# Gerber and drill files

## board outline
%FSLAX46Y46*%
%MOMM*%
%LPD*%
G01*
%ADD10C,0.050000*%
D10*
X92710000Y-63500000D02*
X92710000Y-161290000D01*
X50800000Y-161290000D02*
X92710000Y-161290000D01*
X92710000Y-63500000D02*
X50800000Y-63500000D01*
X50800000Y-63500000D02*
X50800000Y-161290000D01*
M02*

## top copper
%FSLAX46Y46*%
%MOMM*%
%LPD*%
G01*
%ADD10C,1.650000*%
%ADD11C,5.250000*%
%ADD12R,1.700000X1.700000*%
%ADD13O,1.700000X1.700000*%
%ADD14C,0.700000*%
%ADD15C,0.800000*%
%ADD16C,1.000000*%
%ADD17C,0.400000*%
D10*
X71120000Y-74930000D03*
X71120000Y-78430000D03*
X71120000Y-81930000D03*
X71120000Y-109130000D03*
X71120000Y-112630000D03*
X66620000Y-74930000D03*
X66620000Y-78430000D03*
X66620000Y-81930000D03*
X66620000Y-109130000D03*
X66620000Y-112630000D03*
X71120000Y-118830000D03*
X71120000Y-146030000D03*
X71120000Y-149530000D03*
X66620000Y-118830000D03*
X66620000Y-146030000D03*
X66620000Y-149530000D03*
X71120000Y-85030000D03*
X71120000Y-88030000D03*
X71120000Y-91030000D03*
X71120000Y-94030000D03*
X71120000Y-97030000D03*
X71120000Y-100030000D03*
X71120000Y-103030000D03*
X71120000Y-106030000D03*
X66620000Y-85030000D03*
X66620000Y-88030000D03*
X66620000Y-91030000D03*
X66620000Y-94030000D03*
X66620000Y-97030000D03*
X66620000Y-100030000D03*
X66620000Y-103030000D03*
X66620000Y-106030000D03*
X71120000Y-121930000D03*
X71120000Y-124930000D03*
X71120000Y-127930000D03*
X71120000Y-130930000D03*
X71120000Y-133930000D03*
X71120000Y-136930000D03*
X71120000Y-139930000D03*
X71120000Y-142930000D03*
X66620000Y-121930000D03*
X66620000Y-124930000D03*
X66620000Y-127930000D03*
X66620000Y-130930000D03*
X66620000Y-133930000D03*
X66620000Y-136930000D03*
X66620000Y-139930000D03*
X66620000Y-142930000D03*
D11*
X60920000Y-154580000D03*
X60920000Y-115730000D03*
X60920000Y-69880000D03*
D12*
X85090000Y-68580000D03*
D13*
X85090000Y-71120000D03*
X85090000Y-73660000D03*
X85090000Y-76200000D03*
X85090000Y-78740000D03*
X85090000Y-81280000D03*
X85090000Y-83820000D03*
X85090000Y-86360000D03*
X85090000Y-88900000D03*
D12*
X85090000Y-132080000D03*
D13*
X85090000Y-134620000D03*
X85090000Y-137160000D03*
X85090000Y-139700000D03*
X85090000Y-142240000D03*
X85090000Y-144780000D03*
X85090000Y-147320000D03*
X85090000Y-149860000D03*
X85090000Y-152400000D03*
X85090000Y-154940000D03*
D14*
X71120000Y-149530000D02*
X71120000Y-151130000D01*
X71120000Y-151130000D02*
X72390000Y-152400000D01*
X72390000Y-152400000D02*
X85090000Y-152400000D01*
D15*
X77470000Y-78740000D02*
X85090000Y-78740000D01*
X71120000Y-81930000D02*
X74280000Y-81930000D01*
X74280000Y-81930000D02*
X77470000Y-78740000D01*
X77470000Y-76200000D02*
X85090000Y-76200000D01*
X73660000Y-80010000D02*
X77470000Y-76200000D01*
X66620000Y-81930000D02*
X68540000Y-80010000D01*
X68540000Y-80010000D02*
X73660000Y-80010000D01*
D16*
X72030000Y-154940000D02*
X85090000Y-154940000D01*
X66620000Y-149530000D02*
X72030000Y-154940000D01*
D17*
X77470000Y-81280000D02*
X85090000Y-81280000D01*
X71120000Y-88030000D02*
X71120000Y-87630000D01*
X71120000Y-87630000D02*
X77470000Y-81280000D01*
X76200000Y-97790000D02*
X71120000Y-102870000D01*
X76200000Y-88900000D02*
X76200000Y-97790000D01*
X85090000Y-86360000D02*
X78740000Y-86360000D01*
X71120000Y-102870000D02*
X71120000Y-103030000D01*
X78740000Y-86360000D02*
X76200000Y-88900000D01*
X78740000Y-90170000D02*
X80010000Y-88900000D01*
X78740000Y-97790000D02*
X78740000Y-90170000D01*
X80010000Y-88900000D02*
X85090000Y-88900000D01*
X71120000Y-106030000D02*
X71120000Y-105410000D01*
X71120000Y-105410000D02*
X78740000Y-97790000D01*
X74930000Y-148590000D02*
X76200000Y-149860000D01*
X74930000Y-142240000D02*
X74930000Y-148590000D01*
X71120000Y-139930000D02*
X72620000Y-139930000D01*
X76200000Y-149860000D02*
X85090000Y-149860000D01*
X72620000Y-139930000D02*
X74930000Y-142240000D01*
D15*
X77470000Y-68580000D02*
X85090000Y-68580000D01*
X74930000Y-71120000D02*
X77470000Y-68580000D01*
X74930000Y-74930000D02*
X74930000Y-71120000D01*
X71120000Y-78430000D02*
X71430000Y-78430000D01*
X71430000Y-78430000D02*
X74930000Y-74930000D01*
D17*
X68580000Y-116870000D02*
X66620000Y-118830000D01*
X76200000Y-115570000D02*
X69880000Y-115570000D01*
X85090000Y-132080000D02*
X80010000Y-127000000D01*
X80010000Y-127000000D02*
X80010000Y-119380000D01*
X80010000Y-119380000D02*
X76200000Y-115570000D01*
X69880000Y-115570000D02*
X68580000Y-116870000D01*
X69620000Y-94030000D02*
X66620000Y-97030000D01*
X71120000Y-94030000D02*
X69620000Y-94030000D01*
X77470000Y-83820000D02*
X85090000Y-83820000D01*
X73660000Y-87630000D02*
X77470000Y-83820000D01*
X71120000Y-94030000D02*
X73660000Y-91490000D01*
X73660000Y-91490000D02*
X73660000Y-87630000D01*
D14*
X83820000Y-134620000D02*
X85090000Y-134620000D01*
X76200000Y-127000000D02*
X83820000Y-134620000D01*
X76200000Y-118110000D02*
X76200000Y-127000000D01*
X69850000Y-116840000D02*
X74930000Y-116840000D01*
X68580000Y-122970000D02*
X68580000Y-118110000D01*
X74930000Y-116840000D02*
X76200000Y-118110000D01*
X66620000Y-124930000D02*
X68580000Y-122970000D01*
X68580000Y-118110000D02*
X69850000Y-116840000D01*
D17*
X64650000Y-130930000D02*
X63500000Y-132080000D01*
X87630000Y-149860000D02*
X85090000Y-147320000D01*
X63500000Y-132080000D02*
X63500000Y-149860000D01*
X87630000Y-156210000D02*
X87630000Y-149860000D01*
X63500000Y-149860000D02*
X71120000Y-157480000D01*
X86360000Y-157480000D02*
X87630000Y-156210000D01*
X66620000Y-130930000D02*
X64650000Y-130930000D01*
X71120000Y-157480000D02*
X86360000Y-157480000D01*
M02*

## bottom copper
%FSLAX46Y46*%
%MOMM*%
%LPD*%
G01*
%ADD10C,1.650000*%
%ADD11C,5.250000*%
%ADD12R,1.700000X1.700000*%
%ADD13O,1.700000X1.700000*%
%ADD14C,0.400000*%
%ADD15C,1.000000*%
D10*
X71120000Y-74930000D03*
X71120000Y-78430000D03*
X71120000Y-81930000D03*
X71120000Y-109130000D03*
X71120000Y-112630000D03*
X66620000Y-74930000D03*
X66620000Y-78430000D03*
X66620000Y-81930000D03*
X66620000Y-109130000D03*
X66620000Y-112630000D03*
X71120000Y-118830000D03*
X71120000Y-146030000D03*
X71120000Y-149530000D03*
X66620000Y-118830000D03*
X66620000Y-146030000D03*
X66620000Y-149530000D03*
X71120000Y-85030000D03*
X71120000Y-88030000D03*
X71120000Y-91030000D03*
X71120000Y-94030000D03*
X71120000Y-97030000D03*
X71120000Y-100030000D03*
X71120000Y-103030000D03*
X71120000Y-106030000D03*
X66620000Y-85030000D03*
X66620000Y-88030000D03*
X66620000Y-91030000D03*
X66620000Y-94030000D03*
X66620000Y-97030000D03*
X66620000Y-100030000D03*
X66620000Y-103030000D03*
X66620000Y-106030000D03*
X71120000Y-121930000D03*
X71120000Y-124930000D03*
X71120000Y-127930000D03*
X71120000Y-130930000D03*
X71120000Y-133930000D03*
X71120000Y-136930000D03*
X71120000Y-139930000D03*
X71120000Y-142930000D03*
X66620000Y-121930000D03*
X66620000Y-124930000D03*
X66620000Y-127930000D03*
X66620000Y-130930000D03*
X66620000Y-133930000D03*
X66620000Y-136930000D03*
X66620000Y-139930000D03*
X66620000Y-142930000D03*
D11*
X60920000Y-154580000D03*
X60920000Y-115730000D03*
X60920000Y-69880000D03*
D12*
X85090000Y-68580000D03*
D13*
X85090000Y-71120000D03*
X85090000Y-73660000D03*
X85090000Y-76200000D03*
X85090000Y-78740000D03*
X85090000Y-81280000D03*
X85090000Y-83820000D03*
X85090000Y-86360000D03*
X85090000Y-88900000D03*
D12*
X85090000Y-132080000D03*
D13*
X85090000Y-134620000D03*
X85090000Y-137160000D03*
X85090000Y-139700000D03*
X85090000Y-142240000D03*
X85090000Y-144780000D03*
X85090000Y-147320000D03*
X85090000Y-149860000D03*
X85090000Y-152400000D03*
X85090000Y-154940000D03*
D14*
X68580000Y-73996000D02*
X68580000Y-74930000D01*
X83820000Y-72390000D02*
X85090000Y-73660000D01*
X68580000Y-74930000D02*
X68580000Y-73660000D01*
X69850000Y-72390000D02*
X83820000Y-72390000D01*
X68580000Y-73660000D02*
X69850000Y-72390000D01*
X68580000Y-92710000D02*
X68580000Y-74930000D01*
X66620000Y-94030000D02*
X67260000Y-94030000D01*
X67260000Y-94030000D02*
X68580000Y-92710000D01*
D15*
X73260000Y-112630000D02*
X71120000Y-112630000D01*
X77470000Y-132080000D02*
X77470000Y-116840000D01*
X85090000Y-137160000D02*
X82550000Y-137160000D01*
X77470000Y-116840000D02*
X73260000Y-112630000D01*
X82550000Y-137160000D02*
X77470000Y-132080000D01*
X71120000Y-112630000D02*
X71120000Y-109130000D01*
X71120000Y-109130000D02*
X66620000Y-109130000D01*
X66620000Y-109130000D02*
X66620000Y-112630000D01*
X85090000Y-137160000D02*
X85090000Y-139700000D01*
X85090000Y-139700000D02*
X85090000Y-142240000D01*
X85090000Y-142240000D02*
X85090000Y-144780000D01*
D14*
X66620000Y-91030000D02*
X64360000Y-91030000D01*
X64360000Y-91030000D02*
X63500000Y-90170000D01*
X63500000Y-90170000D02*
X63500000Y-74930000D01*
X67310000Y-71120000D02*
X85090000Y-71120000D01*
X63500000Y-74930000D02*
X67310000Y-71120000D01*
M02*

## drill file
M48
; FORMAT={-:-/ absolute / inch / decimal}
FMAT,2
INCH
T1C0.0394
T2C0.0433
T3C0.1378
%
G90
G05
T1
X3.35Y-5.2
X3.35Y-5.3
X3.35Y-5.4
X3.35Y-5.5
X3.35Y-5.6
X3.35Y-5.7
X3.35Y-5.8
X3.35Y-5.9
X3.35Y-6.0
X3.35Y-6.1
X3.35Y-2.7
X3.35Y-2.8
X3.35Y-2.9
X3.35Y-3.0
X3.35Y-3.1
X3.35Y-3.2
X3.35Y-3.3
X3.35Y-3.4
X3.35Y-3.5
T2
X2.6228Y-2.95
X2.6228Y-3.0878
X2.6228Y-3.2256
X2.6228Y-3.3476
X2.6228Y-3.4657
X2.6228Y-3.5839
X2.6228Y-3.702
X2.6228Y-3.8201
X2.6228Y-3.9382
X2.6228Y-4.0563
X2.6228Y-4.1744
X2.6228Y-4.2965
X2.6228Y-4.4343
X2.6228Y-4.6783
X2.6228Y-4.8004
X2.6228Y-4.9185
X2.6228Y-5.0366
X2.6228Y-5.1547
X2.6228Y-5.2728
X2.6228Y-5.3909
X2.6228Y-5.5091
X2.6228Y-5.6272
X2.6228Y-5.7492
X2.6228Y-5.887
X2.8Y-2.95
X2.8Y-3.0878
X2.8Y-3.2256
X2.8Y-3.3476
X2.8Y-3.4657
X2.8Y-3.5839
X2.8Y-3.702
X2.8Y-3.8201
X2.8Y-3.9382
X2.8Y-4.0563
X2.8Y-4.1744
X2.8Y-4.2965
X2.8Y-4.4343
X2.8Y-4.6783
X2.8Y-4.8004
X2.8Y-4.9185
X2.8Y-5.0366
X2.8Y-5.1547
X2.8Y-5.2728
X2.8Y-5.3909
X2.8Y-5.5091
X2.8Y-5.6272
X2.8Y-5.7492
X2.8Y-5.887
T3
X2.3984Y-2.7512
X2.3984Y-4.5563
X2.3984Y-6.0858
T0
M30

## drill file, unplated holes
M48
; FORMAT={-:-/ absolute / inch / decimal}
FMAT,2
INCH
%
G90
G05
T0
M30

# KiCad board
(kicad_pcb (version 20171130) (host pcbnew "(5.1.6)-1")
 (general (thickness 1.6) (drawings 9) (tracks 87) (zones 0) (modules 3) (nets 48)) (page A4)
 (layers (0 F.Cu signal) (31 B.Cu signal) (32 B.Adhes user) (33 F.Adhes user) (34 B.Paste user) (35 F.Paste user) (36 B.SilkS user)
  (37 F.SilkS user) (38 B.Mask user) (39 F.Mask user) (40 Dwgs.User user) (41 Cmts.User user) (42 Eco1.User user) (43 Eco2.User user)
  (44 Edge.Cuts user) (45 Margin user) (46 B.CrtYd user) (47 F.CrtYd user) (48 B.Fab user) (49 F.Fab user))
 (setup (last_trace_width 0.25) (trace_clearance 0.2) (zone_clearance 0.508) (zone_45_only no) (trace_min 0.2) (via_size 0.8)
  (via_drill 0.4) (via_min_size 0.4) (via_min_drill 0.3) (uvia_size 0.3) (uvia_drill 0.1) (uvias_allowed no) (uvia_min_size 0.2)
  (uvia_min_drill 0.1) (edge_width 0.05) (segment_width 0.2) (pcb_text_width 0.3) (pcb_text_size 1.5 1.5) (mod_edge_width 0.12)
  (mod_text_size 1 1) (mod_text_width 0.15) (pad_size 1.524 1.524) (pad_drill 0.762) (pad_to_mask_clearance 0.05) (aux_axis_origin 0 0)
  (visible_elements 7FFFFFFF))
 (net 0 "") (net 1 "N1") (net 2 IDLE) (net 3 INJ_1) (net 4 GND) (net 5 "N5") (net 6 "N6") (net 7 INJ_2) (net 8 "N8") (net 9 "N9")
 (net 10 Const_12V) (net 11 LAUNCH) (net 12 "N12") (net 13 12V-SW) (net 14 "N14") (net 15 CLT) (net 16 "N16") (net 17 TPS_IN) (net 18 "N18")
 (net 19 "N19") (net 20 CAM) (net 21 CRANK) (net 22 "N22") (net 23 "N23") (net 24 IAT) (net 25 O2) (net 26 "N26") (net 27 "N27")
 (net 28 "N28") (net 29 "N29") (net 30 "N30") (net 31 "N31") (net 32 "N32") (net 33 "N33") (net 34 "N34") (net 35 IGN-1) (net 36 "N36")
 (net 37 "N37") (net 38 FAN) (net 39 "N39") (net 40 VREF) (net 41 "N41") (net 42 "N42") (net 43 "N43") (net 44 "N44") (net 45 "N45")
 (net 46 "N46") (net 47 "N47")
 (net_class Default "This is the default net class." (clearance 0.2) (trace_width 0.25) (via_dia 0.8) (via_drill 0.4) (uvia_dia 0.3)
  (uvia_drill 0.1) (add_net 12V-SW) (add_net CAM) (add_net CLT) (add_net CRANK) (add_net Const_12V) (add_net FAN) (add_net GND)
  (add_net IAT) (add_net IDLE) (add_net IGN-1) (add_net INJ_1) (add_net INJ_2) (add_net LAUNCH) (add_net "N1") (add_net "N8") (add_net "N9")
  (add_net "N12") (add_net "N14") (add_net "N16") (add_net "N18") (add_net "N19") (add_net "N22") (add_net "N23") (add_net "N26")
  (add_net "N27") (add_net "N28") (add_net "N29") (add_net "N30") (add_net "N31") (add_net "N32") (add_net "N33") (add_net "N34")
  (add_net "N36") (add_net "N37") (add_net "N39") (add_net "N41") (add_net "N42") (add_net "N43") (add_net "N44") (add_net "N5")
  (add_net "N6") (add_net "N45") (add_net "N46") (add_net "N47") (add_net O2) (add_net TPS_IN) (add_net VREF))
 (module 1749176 (layer F.Cu) (at 71.12 74.93 180)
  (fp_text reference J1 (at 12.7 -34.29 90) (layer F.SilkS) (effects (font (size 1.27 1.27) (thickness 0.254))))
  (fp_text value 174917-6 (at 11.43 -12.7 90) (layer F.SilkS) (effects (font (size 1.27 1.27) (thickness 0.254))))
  (pad 1 thru_hole circle (at 0 0 270) (size 1.65 1.65) (drill 1.1) (layers *.Cu *.Mask F.SilkS) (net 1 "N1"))
  (pad 2 thru_hole circle (at 0 -3.5 270) (size 1.65 1.65) (drill 1.1) (layers *.Cu *.Mask F.SilkS) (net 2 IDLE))
  (pad 3 thru_hole circle (at 0 -7 270) (size 1.65 1.65) (drill 1.1) (layers *.Cu *.Mask F.SilkS) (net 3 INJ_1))
  (pad 4 thru_hole circle (at 0 -34.2 270) (size 1.65 1.65) (drill 1.1) (layers *.Cu *.Mask F.SilkS) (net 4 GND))
  (pad 5 thru_hole circle (at 0 -37.7 270) (size 1.65 1.65) (drill 1.1) (layers *.Cu *.Mask F.SilkS) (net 4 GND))
  (pad 6 thru_hole circle (at 4.5 0 270) (size 1.65 1.65) (drill 1.1) (layers *.Cu *.Mask F.SilkS) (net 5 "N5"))
  (pad 7 thru_hole circle (at 4.5 -3.5 270) (size 1.65 1.65) (drill 1.1) (layers *.Cu *.Mask F.SilkS) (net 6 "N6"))
  (pad 8 thru_hole circle (at 4.5 -7 270) (size 1.65 1.65) (drill 1.1) (layers *.Cu *.Mask F.SilkS) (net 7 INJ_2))
  (pad 9 thru_hole circle (at 4.5 -34.2 270) (size 1.65 1.65) (drill 1.1) (layers *.Cu *.Mask F.SilkS) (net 4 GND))
  (pad 10 thru_hole circle (at 4.5 -37.7 270) (size 1.65 1.65) (drill 1.1) (layers *.Cu *.Mask F.SilkS) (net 4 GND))
  (pad 11 thru_hole circle (at 0 -43.9 270) (size 1.65 1.65) (drill 1.1) (layers *.Cu *.Mask F.SilkS) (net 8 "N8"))
  (pad 12 thru_hole circle (at 0 -71.1 270) (size 1.65 1.65) (drill 1.1) (layers *.Cu *.Mask F.SilkS) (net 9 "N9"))
  (pad 13 thru_hole circle (at 0 -74.6 270) (size 1.65 1.65) (drill 1.1) (layers *.Cu *.Mask F.SilkS) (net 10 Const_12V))
  (pad 14 thru_hole circle (at 4.5 -43.9 270) (size 1.65 1.65) (drill 1.1) (layers *.Cu *.Mask F.SilkS) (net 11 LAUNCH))
  (pad 15 thru_hole circle (at 4.5 -71.1 270) (size 1.65 1.65) (drill 1.1) (layers *.Cu *.Mask F.SilkS) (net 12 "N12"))
  (pad 16 thru_hole circle (at 4.5 -74.6 270) (size 1.65 1.65) (drill 1.1) (layers *.Cu *.Mask F.SilkS) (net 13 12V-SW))
  (pad 17 thru_hole circle (at 0 -10.1 270) (size 1.65 1.65) (drill 1.1) (layers *.Cu *.Mask F.SilkS) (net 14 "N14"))
  (pad 18 thru_hole circle (at 0 -13.1 270) (size 1.65 1.65) (drill 1.1) (layers *.Cu *.Mask F.SilkS) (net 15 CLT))
  (pad 19 thru_hole circle (at 0 -16.1 270) (size 1.65 1.65) (drill 1.1) (layers *.Cu *.Mask F.SilkS) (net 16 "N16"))
  (pad 20 thru_hole circle (at 0 -19.1 270) (size 1.65 1.65) (drill 1.1) (layers *.Cu *.Mask F.SilkS) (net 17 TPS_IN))
  (pad 21 thru_hole circle (at 0 -22.1 270) (size 1.65 1.65) (drill 1.1) (layers *.Cu *.Mask F.SilkS) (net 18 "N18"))
  (pad 22 thru_hole circle (at 0 -25.1 270) (size 1.65 1.65) (drill 1.1) (layers *.Cu *.Mask F.SilkS) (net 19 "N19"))
  (pad 23 thru_hole circle (at 0 -28.1 270) (size 1.65 1.65) (drill 1.1) (layers *.Cu *.Mask F.SilkS) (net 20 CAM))
  (pad 24 thru_hole circle (at 0 -31.1 270) (size 1.65 1.65) (drill 1.1) (layers *.Cu *.Mask F.SilkS) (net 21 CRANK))
  (pad 25 thru_hole circle (at 4.5 -10.1 270) (size 1.65 1.65) (drill 1.1) (layers *.Cu *.Mask F.SilkS) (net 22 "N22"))
  (pad 26 thru_hole circle (at 4.5 -13.1 270) (size 1.65 1.65) (drill 1.1) (layers *.Cu *.Mask F.SilkS) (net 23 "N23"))
  (pad 27 thru_hole circle (at 4.5 -16.1 270) (size 1.65 1.65) (drill 1.1) (layers *.Cu *.Mask F.SilkS) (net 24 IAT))
  (pad 28 thru_hole circle (at 4.5 -19.1 270) (size 1.65 1.65) (drill 1.1) (layers *.Cu *.Mask F.SilkS) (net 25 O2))
  (pad 29 thru_hole circle (at 4.5 -22.1 270) (size 1.65 1.65) (drill 1.1) (layers *.Cu *.Mask F.SilkS) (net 17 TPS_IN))
  (pad 30 thru_hole circle (at 4.5 -25.1 270) (size 1.65 1.65) (drill 1.1) (layers *.Cu *.Mask F.SilkS) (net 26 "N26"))
  (pad 31 thru_hole circle (at 4.5 -28.1 270) (size 1.65 1.65) (drill 1.1) (layers *.Cu *.Mask F.SilkS) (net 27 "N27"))
  (pad 32 thru_hole circle (at 4.5 -31.1 270) (size 1.65 1.65) (drill 1.1) (layers *.Cu *.Mask F.SilkS) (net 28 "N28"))
  (pad 33 thru_hole circle (at 0 -47 270) (size 1.65 1.65) (drill 1.1) (layers *.Cu *.Mask F.SilkS) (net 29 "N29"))
  (pad 34 thru_hole circle (at 0 -50 270) (size 1.65 1.65) (drill 1.1) (layers *.Cu *.Mask F.SilkS) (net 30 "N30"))
  (pad 35 thru_hole circle (at 0 -53 270) (size 1.65 1.65) (drill 1.1) (layers *.Cu *.Mask F.SilkS) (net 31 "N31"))
  (pad 36 thru_hole circle (at 0 -56 270) (size 1.65 1.65) (drill 1.1) (layers *.Cu *.Mask F.SilkS) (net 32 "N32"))
  (pad 37 thru_hole circle (at 0 -59 270) (size 1.65 1.65) (drill 1.1) (layers *.Cu *.Mask F.SilkS) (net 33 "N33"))
  (pad 38 thru_hole circle (at 0 -62 270) (size 1.65 1.65) (drill 1.1) (layers *.Cu *.Mask F.SilkS) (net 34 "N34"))
  (pad 39 thru_hole circle (at 0 -65 270) (size 1.65 1.65) (drill 1.1) (layers *.Cu *.Mask F.SilkS) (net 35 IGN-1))
  (pad 40 thru_hole circle (at 0 -68 270) (size 1.65 1.65) (drill 1.1) (layers *.Cu *.Mask F.SilkS) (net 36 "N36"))
  (pad 41 thru_hole circle (at 4.5 -47 270) (size 1.65 1.65) (drill 1.1) (layers *.Cu *.Mask F.SilkS) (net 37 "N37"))
  (pad 42 thru_hole circle (at 4.5 -50 270) (size 1.65 1.65) (drill 1.1) (layers *.Cu *.Mask F.SilkS) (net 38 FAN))
  (pad 43 thru_hole circle (at 4.5 -53 270) (size 1.65 1.65) (drill 1.1) (layers *.Cu *.Mask F.SilkS) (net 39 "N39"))
  (pad 44 thru_hole circle (at 4.5 -56 270) (size 1.65 1.65) (drill 1.1) (layers *.Cu *.Mask F.SilkS) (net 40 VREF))
  (pad 45 thru_hole circle (at 4.5 -59 270) (size 1.65 1.65) (drill 1.1) (layers *.Cu *.Mask F.SilkS) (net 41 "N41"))
  (pad 46 thru_hole circle (at 4.5 -62 270) (size 1.65 1.65) (drill 1.1) (layers *.Cu *.Mask F.SilkS) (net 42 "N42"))
  (pad 47 thru_hole circle (at 4.5 -65 270) (size 1.65 1.65) (drill 1.1) (layers *.Cu *.Mask F.SilkS) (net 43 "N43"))
  (pad 48 thru_hole circle (at 4.5 -68 270) (size 1.65 1.65) (drill 1.1) (layers *.Cu *.Mask F.SilkS) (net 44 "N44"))
  (pad MH1 thru_hole circle (at 10.2 -79.65 270) (size 5.25 5.25) (drill 3.5) (layers *.Cu *.Mask F.SilkS) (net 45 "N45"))
  (pad MH2 thru_hole circle (at 10.2 -40.8 270) (size 5.25 5.25) (drill 3.5) (layers *.Cu *.Mask F.SilkS) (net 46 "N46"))
  (pad MH3 thru_hole circle (at 10.2 5.05 270) (size 5.25 5.25) (drill 3.5) (layers *.Cu *.Mask F.SilkS) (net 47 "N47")))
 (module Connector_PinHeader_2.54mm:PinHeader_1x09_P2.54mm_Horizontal (layer F.Cu) (at 85.09 68.58)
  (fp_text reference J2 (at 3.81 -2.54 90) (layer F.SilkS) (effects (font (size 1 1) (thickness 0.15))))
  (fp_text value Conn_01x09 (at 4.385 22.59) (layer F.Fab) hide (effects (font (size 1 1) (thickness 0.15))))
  (pad 1 thru_hole rect (at 0 0) (size 1.7 1.7) (drill 1) (layers *.Cu *.Mask) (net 2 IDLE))
  (pad 2 thru_hole oval (at 0 2.54) (size 1.7 1.7) (drill 1) (layers *.Cu *.Mask) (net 24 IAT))
  (pad 3 thru_hole oval (at 0 5.08) (size 1.7 1.7) (drill 1) (layers *.Cu *.Mask) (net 25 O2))
  (pad 4 thru_hole oval (at 0 7.62) (size 1.7 1.7) (drill 1) (layers *.Cu *.Mask) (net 7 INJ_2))
  (pad 5 thru_hole oval (at 0 10.16) (size 1.7 1.7) (drill 1) (layers *.Cu *.Mask) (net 3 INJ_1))
  (pad 6 thru_hole oval (at 0 12.7) (size 1.7 1.7) (drill 1) (layers *.Cu *.Mask) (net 15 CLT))
  (pad 7 thru_hole oval (at 0 15.24) (size 1.7 1.7) (drill 1) (layers *.Cu *.Mask) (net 17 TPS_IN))
  (pad 8 thru_hole oval (at 0 17.78) (size 1.7 1.7) (drill 1) (layers *.Cu *.Mask) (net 20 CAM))
  (pad 9 thru_hole oval (at 0 20.32) (size 1.7 1.7) (drill 1) (layers *.Cu *.Mask) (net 21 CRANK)))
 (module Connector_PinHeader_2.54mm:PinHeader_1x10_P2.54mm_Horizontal (layer F.Cu) (at 85.09 132.08)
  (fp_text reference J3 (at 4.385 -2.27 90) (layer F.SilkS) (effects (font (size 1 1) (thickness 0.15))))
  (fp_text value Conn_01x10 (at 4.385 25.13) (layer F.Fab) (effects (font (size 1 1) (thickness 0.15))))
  (pad 1 thru_hole rect (at 0 0) (size 1.7 1.7) (drill 1) (layers *.Cu *.Mask) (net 11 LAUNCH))
  (pad 2 thru_hole oval (at 0 2.54) (size 1.7 1.7) (drill 1) (layers *.Cu *.Mask) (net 38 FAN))
  (pad 3 thru_hole oval (at 0 5.08) (size 1.7 1.7) (drill 1) (layers *.Cu *.Mask) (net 4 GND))
  (pad 4 thru_hole oval (at 0 7.62) (size 1.7 1.7) (drill 1) (layers *.Cu *.Mask) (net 4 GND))
  (pad 5 thru_hole oval (at 0 10.16) (size 1.7 1.7) (drill 1) (layers *.Cu *.Mask) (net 4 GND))
  (pad 6 thru_hole oval (at 0 12.7) (size 1.7 1.7) (drill 1) (layers *.Cu *.Mask) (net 4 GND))
  (pad 7 thru_hole oval (at 0 15.24) (size 1.7 1.7) (drill 1) (layers *.Cu *.Mask) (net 40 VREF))
  (pad 8 thru_hole oval (at 0 17.78) (size 1.7 1.7) (drill 1) (layers *.Cu *.Mask) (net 35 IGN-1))
  (pad 9 thru_hole oval (at 0 20.32) (size 1.7 1.7) (drill 1) (layers *.Cu *.Mask) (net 10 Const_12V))
  (pad 10 thru_hole oval (at 0 22.86) (size 1.7 1.7) (drill 1) (layers *.Cu *.Mask) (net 13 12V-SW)))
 (gr_line (start 92.71 63.5) (end 92.71 161.29) (layer Edge.Cuts) (width 0.05))
 (gr_line (start 50.8 161.29) (end 92.71 161.29) (layer Edge.Cuts) (width 0.05))
 (gr_line (start 92.71 63.5) (end 50.8 63.5) (layer Edge.Cuts) (width 0.05))
 (gr_line (start 50.8 63.5) (end 50.8 161.29) (layer Edge.Cuts) (width 0.05))
 (segment (start 71.12 149.53) (end 71.12 151.13) (width 0.7) (layer F.Cu) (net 10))
 (segment (start 71.12 151.13) (end 72.39 152.4) (width 0.7) (layer F.Cu) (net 10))
 (segment (start 72.39 152.4) (end 85.09 152.4) (width 0.7) (layer F.Cu) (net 10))
 (segment (start 77.47 78.74) (end 85.09 78.74) (width 0.8) (layer F.Cu) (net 3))
 (segment (start 71.12 81.93) (end 74.28 81.93) (width 0.8) (layer F.Cu) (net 3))
 (segment (start 74.28 81.93) (end 77.47 78.74) (width 0.8) (layer F.Cu) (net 3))
 (segment (start 77.47 76.2) (end 85.09 76.2) (width 0.8) (layer F.Cu) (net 7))
 (segment (start 73.66 80.01) (end 77.47 76.2) (width 0.8) (layer F.Cu) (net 7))
 (segment (start 66.62 81.93) (end 68.54 80.01) (width 0.8) (layer F.Cu) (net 7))
 (segment (start 68.54 80.01) (end 73.66 80.01) (width 0.8) (layer F.Cu) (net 7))
 (segment (start 68.58 73.996) (end 68.58 74.93) (width 0.4) (layer B.Cu) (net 25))
 (segment (start 83.82 72.39) (end 85.09 73.66) (width 0.4) (layer B.Cu) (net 25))
 (segment (start 68.58 74.93) (end 68.58 73.66) (width 0.4) (layer B.Cu) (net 25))
 (segment (start 69.85 72.39) (end 83.82 72.39) (width 0.4) (layer B.Cu) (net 25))
 (segment (start 68.58 73.66) (end 69.85 72.39) (width 0.4) (layer B.Cu) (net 25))
 (segment (start 68.58 92.71) (end 68.58 74.93) (width 0.4) (layer B.Cu) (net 25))
 (segment (start 66.62 94.03) (end 67.26 94.03) (width 0.4) (layer B.Cu) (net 25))
 (segment (start 67.26 94.03) (end 68.58 92.71) (width 0.4) (layer B.Cu) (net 25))
 (segment (start 73.26 112.63) (end 71.12 112.63) (width 1) (layer B.Cu) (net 4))
 (segment (start 77.47 132.08) (end 77.47 116.84) (width 1) (layer B.Cu) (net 4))
 (segment (start 85.09 137.16) (end 82.55 137.16) (width 1) (layer B.Cu) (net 4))
 (segment (start 77.47 116.84) (end 73.26 112.63) (width 1) (layer B.Cu) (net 4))
 (segment (start 82.55 137.16) (end 77.47 132.08) (width 1) (layer B.Cu) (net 4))
 (segment (start 71.12 112.63) (end 71.12 109.13) (width 1) (layer B.Cu) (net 4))
 (segment (start 71.12 109.13) (end 66.62 109.13) (width 1) (layer B.Cu) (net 4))
 (segment (start 66.62 109.13) (end 66.62 112.63) (width 1) (layer B.Cu) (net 4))
 (segment (start 85.09 137.16) (end 85.09 139.7) (width 1) (layer B.Cu) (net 4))
 (segment (start 85.09 139.7) (end 85.09 142.24) (width 1) (layer B.Cu) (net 4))
 (segment (start 85.09 142.24) (end 85.09 144.78) (width 1) (layer B.Cu) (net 4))
 (segment (start 72.03 154.94) (end 85.09 154.94) (width 1) (layer F.Cu) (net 13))
 (segment (start 66.62 149.53) (end 72.03 154.94) (width 1) (layer F.Cu) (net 13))
 (segment (start 77.47 81.28) (end 85.09 81.28) (width 0.4) (layer F.Cu) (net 15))
 (segment (start 71.12 88.03) (end 71.12 87.63) (width 0.4) (layer F.Cu) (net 15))
 (segment (start 71.12 87.63) (end 77.47 81.28) (width 0.4) (layer F.Cu) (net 15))
 (segment (start 76.2 97.79) (end 71.12 102.87) (width 0.4) (layer F.Cu) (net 20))
 (segment (start 76.2 88.9) (end 76.2 97.79) (width 0.4) (layer F.Cu) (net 20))
 (segment (start 85.09 86.36) (end 78.74 86.36) (width 0.4) (layer F.Cu) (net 20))
 (segment (start 71.12 102.87) (end 71.12 103.03) (width 0.4) (layer F.Cu) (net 20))
 (segment (start 78.74 86.36) (end 76.2 88.9) (width 0.4) (layer F.Cu) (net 20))
 (segment (start 78.74 90.17) (end 80.01 88.9) (width 0.4) (layer F.Cu) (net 21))
 (segment (start 78.74 97.79) (end 78.74 90.17) (width 0.4) (layer F.Cu) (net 21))
 (segment (start 80.01 88.9) (end 85.09 88.9) (width 0.4) (layer F.Cu) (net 21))
 (segment (start 71.12 106.03) (end 71.12 105.41) (width 0.4) (layer F.Cu) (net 21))
 (segment (start 71.12 105.41) (end 78.74 97.79) (width 0.4) (layer F.Cu) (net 21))
 (segment (start 74.93 148.59) (end 76.2 149.86) (width 0.4) (layer F.Cu) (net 35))
 (segment (start 74.93 142.24) (end 74.93 148.59) (width 0.4) (layer F.Cu) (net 35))
 (segment (start 71.12 139.93) (end 72.62 139.93) (width 0.4) (layer F.Cu) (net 35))
 (segment (start 76.2 149.86) (end 85.09 149.86) (width 0.4) (layer F.Cu) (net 35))
 (segment (start 72.62 139.93) (end 74.93 142.24) (width 0.4) (layer F.Cu) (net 35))
 (segment (start 77.47 68.58) (end 85.09 68.58) (width 0.8) (layer F.Cu) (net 2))
 (segment (start 74.93 71.12) (end 77.47 68.58) (width 0.8) (layer F.Cu) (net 2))
 (segment (start 74.93 74.93) (end 74.93 71.12) (width 0.8) (layer F.Cu) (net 2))
 (segment (start 71.12 78.43) (end 71.43 78.43) (width 0.8) (layer F.Cu) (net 2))
 (segment (start 71.43 78.43) (end 74.93 74.93) (width 0.8) (layer F.Cu) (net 2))
 (segment (start 68.58 116.87) (end 66.62 118.83) (width 0.4) (layer F.Cu) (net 11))
 (segment (start 76.2 115.57) (end 69.88 115.57) (width 0.4) (layer F.Cu) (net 11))
 (segment (start 85.09 132.08) (end 80.01 127) (width 0.4) (layer F.Cu) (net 11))
 (segment (start 80.01 127) (end 80.01 119.38) (width 0.4) (layer F.Cu) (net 11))
 (segment (start 80.01 119.38) (end 76.2 115.57) (width 0.4) (layer F.Cu) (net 11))
 (segment (start 69.88 115.57) (end 68.58 116.87) (width 0.4) (layer F.Cu) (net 11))
 (segment (start 69.62 94.03) (end 66.62 97.03) (width 0.4) (layer F.Cu) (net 17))
 (segment (start 71.12 94.03) (end 69.62 94.03) (width 0.4) (layer F.Cu) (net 17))
 (segment (start 77.47 83.82) (end 85.09 83.82) (width 0.4) (layer F.Cu) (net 17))
 (segment (start 73.66 87.63) (end 77.47 83.82) (width 0.4) (layer F.Cu) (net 17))
 (segment (start 71.12 94.03) (end 73.66 91.49) (width 0.4) (layer F.Cu) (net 17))
 (segment (start 73.66 91.49) (end 73.66 87.63) (width 0.4) (layer F.Cu) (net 17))
 (segment (start 66.62 91.03) (end 64.36 91.03) (width 0.4) (layer B.Cu) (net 24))
 (segment (start 64.36 91.03) (end 63.5 90.17) (width 0.4) (layer B.Cu) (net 24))
 (segment (start 63.5 90.17) (end 63.5 74.93) (width 0.4) (layer B.Cu) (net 24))
 (segment (start 67.31 71.12) (end 85.09 71.12) (width 0.4) (layer B.Cu) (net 24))
 (segment (start 63.5 74.93) (end 67.31 71.12) (width 0.4) (layer B.Cu) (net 24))
 (segment (start 83.82 134.62) (end 85.09 134.62) (width 0.7) (layer F.Cu) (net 38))
 (segment (start 76.2 127) (end 83.82 134.62) (width 0.7) (layer F.Cu) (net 38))
 (segment (start 76.2 118.11) (end 76.2 127) (width 0.7) (layer F.Cu) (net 38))
 (segment (start 69.85 116.84) (end 74.93 116.84) (width 0.7) (layer F.Cu) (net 38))
 (segment (start 68.58 122.97) (end 68.58 118.11) (width 0.7) (layer F.Cu) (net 38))
 (segment (start 74.93 116.84) (end 76.2 118.11) (width 0.7) (layer F.Cu) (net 38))
 (segment (start 66.62 124.93) (end 68.58 122.97) (width 0.7) (layer F.Cu) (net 38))
 (segment (start 68.58 118.11) (end 69.85 116.84) (width 0.7) (layer F.Cu) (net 38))
 (segment (start 64.65 130.93) (end 63.5 132.08) (width 0.4) (layer F.Cu) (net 40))
 (segment (start 87.63 149.86) (end 85.09 147.32) (width 0.4) (layer F.Cu) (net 40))
 (segment (start 63.5 132.08) (end 63.5 149.86) (width 0.4) (layer F.Cu) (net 40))
 (segment (start 87.63 156.21) (end 87.63 149.86) (width 0.4) (layer F.Cu) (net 40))
 (segment (start 63.5 149.86) (end 71.12 157.48) (width 0.4) (layer F.Cu) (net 40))
 (segment (start 86.36 157.48) (end 87.63 156.21) (width 0.4) (layer F.Cu) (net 40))
 (segment (start 66.62 130.93) (end 64.65 130.93) (width 0.4) (layer F.Cu) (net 40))
 (segment (start 71.12 157.48) (end 86.36 157.48) (width 0.4) (layer F.Cu) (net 40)))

